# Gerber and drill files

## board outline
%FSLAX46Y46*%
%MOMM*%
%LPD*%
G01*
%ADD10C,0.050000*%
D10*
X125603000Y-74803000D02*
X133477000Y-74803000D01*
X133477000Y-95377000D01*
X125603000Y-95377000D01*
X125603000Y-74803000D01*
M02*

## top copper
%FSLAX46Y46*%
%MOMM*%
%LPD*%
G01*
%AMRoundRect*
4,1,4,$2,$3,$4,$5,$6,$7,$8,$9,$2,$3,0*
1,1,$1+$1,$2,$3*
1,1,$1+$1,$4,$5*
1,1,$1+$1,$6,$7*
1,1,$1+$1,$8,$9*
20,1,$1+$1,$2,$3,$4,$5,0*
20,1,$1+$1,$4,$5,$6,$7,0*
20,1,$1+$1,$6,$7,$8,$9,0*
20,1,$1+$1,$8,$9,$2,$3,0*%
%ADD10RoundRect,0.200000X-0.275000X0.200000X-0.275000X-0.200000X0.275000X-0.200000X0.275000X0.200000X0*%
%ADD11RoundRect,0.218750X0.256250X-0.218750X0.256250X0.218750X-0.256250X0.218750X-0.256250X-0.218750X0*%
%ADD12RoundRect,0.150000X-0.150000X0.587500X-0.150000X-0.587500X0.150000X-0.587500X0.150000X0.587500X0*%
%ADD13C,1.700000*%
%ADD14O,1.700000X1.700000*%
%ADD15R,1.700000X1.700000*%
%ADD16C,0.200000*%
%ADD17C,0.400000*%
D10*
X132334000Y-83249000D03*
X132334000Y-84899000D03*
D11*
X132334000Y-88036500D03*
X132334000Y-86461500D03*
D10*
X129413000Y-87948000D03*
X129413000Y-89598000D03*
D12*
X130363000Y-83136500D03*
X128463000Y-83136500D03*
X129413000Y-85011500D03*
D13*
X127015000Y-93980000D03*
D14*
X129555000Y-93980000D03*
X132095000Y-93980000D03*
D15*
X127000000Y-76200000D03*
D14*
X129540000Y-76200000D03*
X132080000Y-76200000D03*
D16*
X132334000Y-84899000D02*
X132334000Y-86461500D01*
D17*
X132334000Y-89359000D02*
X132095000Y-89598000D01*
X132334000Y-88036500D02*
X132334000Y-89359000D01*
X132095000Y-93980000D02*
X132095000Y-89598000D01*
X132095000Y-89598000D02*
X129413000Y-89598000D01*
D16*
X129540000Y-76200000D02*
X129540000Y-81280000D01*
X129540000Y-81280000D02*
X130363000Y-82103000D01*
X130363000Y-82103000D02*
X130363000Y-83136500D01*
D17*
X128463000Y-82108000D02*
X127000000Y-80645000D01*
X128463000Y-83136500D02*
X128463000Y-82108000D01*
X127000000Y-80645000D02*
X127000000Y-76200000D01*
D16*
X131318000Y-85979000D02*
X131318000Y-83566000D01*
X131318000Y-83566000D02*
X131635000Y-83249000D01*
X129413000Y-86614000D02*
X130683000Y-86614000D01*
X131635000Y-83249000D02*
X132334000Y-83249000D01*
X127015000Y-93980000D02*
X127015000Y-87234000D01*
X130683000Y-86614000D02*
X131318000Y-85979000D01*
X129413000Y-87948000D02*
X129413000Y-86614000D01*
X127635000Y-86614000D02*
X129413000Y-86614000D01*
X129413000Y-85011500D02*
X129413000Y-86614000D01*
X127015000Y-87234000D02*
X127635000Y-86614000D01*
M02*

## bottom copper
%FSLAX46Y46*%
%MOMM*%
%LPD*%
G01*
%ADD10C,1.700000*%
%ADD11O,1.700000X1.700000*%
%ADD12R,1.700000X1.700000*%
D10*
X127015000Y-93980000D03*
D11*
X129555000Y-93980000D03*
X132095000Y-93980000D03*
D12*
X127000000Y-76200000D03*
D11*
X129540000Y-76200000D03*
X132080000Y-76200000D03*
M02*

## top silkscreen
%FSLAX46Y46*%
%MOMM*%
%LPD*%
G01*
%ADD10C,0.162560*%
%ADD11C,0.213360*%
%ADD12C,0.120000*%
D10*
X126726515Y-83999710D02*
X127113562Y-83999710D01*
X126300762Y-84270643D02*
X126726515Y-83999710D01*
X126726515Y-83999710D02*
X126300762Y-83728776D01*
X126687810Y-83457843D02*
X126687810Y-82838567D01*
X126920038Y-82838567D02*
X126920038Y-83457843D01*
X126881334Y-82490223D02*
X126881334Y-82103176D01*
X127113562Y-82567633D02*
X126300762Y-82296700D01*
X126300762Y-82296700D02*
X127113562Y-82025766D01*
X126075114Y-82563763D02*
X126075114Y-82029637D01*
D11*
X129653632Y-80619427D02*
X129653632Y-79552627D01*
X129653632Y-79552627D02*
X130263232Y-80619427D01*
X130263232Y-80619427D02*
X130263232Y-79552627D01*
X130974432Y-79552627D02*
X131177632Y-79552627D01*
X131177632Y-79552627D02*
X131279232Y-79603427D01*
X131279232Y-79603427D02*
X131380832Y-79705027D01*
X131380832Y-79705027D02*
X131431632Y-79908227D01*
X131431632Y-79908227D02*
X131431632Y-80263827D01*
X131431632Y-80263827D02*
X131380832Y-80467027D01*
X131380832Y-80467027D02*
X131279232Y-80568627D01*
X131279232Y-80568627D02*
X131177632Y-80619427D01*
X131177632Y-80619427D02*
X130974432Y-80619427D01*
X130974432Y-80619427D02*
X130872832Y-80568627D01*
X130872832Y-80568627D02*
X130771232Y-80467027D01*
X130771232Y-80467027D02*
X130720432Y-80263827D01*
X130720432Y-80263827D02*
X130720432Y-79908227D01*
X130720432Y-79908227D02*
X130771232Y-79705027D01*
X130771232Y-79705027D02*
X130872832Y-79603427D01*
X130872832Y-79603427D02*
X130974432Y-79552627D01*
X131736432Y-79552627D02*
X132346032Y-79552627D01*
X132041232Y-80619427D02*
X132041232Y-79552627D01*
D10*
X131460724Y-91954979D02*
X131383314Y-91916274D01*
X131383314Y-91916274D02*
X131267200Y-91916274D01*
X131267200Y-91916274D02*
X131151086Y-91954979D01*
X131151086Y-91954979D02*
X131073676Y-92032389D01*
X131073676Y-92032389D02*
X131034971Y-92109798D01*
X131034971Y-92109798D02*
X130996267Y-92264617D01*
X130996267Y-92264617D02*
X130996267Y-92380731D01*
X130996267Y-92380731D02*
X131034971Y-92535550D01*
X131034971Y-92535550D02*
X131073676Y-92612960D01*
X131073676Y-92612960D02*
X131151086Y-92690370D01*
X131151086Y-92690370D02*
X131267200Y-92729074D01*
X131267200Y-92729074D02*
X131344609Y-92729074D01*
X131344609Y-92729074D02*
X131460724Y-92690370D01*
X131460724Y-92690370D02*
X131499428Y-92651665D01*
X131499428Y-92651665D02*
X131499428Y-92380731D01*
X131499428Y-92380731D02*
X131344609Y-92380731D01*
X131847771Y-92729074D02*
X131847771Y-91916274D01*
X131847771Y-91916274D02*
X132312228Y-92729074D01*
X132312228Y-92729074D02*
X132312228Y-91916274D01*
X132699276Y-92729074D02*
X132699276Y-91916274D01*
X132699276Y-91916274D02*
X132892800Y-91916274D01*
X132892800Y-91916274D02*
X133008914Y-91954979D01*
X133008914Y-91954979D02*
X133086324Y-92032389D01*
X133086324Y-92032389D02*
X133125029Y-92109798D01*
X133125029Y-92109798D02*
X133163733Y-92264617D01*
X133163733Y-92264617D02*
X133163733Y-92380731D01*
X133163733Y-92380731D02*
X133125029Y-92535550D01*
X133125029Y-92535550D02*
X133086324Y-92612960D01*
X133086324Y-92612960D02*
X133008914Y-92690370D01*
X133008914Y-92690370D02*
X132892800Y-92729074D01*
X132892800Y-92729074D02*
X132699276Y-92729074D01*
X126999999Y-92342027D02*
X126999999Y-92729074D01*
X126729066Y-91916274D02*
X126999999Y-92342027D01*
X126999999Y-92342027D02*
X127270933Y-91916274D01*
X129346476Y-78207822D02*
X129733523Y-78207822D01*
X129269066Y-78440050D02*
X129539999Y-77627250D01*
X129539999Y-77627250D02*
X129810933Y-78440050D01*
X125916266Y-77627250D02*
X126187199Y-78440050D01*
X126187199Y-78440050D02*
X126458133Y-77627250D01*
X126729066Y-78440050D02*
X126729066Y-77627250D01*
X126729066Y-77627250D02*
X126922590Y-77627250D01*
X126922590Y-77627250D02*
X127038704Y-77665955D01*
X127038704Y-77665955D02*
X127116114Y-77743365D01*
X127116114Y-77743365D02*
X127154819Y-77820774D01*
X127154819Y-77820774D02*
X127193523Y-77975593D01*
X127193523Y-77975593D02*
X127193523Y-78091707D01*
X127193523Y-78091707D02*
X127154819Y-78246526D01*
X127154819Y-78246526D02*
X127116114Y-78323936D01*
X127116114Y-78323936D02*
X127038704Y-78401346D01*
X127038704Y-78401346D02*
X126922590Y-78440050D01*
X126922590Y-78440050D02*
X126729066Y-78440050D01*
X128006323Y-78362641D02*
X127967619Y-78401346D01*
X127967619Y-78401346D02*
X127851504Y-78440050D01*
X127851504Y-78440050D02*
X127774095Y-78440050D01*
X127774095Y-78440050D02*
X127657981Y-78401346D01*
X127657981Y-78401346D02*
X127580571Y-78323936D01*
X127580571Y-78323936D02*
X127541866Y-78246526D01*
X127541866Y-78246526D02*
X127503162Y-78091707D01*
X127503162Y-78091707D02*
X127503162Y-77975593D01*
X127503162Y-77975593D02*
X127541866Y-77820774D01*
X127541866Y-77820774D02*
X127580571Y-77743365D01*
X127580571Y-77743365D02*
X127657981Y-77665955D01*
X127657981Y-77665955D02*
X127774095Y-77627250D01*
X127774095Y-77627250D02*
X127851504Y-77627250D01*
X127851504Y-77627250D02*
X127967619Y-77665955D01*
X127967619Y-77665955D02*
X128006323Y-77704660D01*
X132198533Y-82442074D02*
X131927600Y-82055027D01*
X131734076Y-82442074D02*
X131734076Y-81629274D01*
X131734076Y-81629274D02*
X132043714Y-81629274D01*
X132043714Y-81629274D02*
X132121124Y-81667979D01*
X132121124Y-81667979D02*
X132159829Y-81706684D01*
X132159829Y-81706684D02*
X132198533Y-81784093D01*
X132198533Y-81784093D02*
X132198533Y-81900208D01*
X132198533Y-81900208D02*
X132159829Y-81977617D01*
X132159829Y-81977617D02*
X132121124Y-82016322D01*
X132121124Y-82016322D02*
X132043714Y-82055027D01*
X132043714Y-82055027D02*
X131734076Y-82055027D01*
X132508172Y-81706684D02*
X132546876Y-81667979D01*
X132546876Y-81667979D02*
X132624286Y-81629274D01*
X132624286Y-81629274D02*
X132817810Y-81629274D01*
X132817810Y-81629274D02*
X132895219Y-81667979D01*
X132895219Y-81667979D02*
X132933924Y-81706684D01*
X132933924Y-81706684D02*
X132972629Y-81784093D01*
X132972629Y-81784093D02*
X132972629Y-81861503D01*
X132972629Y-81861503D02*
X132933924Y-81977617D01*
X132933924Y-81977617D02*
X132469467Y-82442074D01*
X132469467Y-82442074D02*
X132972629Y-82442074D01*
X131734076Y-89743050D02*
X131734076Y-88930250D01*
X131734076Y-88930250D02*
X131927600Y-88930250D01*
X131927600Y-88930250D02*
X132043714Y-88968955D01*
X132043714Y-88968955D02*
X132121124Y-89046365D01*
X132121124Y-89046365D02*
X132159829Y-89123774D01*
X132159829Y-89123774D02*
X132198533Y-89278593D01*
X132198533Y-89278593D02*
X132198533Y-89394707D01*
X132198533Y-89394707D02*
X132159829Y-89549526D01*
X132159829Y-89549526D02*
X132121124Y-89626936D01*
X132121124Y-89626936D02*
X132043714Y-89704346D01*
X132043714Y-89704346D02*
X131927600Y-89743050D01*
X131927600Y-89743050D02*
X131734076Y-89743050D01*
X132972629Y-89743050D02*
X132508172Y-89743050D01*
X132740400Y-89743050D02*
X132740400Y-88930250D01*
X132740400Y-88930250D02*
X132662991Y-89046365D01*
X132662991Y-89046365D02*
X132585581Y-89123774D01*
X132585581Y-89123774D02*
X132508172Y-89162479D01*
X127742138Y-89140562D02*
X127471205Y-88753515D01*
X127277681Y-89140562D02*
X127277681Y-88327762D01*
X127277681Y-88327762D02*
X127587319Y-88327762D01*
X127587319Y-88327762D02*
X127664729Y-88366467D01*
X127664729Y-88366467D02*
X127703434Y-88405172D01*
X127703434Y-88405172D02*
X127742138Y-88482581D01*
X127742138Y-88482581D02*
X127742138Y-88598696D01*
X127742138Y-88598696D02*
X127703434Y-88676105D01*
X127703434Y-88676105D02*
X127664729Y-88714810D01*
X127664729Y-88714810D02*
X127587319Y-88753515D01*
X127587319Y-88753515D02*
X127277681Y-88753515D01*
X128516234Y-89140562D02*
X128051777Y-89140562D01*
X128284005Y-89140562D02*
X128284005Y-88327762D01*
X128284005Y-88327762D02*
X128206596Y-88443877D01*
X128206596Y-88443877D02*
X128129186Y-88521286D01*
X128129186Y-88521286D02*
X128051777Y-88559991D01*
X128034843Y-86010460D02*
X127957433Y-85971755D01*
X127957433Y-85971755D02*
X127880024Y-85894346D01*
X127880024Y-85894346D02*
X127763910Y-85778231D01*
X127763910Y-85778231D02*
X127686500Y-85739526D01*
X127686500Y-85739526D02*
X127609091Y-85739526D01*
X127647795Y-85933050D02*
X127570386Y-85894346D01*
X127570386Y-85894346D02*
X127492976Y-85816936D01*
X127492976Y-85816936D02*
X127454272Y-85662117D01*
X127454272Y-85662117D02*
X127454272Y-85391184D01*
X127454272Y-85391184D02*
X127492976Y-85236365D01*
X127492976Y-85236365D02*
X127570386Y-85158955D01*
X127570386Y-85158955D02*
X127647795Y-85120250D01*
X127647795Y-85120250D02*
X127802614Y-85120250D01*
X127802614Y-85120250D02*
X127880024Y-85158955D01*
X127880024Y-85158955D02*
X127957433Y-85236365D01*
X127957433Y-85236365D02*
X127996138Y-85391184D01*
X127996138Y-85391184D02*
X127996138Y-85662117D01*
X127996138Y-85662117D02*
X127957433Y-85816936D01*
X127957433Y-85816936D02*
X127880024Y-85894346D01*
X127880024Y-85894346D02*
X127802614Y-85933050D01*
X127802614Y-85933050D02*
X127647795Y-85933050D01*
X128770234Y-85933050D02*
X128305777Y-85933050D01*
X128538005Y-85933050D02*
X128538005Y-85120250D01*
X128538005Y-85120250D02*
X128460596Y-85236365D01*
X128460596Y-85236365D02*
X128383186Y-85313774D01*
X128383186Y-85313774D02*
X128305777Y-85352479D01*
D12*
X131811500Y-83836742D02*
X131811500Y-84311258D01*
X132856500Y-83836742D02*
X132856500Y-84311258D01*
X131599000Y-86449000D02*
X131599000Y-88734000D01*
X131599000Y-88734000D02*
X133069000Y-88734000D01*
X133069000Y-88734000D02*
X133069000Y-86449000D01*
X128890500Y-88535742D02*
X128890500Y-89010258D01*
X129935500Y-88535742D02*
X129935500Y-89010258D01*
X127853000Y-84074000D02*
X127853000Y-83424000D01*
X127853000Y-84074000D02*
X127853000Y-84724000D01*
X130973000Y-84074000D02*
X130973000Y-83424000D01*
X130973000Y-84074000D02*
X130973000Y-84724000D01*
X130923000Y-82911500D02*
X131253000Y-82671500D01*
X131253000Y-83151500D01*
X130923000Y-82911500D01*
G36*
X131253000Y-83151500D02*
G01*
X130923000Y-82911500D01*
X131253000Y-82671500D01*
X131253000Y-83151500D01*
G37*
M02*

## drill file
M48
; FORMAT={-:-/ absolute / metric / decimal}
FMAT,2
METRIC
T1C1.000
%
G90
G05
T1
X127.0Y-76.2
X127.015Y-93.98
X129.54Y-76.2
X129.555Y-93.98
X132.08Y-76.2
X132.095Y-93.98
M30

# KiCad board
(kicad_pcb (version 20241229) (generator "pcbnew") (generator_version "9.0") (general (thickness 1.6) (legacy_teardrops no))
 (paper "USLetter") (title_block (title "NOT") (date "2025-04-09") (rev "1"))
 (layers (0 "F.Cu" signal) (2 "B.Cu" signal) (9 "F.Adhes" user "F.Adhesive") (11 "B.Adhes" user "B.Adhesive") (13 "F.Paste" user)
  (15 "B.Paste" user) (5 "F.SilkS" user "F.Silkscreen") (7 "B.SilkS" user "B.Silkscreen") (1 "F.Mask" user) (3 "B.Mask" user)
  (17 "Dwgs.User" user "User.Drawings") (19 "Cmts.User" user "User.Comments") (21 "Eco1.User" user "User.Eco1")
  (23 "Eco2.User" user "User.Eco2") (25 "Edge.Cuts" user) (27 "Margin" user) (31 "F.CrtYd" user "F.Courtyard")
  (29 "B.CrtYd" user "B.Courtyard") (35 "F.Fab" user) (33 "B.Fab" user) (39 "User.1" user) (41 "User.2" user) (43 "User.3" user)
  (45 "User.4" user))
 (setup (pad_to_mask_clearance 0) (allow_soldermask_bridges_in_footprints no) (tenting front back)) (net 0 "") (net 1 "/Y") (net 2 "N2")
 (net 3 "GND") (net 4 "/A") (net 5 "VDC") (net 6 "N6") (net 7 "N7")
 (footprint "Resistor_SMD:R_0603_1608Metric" (layer "F.Cu") (at 132.334 84.074 -90)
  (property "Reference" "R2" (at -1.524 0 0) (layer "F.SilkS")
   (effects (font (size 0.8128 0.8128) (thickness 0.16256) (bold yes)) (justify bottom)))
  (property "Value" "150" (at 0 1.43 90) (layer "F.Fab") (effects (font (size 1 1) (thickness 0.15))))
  (fp_line (start -0.237258 0.5225) (end 0.237258 0.5225) (stroke (width 0.12) (type solid)) (layer "F.SilkS"))
  (fp_line (start -0.237258 -0.5225) (end 0.237258 -0.5225) (stroke (width 0.12) (type solid)) (layer "F.SilkS"))
  (pad "1" smd roundrect (at -0.825 0 270) (size 0.8 0.95) (layers "F.Cu" "F.Mask" "F.Paste") (roundrect_rratio 0.25) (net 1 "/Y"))
  (pad "2" smd roundrect (at 0.825 0 270) (size 0.8 0.95) (layers "F.Cu" "F.Mask" "F.Paste") (roundrect_rratio 0.25) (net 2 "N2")))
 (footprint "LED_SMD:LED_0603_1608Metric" (layer "F.Cu") (at 132.334 87.249 90)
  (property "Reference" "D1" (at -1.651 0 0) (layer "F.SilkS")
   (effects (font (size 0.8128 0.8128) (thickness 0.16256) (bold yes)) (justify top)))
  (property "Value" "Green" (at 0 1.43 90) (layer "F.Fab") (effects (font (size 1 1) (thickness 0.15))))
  (fp_line (start 0.8 -0.735) (end -1.485 -0.735) (stroke (width 0.12) (type solid)) (layer "F.SilkS"))
  (fp_line (start -1.485 -0.735) (end -1.485 0.735) (stroke (width 0.12) (type solid)) (layer "F.SilkS"))
  (fp_line (start -1.485 0.735) (end 0.8 0.735) (stroke (width 0.12) (type solid)) (layer "F.SilkS"))
  (pad "1" smd roundrect (at -0.7875 0 90) (size 0.875 0.95) (layers "F.Cu" "F.Mask" "F.Paste") (roundrect_rratio 0.25) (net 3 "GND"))
  (pad "2" smd roundrect (at 0.7875 0 90) (size 0.875 0.95) (layers "F.Cu" "F.Mask" "F.Paste") (roundrect_rratio 0.25) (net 2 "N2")))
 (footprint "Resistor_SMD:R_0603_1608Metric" (layer "F.Cu") (at 129.413 88.773 -90)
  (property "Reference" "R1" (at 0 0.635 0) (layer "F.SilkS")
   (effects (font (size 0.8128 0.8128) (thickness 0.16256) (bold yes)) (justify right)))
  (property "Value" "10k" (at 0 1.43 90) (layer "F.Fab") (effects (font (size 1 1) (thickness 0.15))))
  (fp_line (start -0.237258 0.5225) (end 0.237258 0.5225) (stroke (width 0.12) (type solid)) (layer "F.SilkS"))
  (fp_line (start -0.237258 -0.5225) (end 0.237258 -0.5225) (stroke (width 0.12) (type solid)) (layer "F.SilkS"))
  (pad "1" smd roundrect (at -0.825 0 270) (size 0.8 0.95) (layers "F.Cu" "F.Mask" "F.Paste") (roundrect_rratio 0.25) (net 1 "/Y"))
  (pad "2" smd roundrect (at 0.825 0 270) (size 0.8 0.95) (layers "F.Cu" "F.Mask" "F.Paste") (roundrect_rratio 0.25) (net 3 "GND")))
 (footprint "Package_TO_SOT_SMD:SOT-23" (layer "F.Cu") (at 129.413 84.074 -90)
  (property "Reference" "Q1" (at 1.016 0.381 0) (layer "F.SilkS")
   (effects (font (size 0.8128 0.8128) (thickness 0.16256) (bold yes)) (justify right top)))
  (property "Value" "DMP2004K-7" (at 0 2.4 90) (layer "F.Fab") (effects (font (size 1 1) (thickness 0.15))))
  (fp_line (start 0 1.56) (end -0.65 1.56) (stroke (width 0.12) (type solid)) (layer "F.SilkS"))
  (fp_line (start 0 1.56) (end 0.65 1.56) (stroke (width 0.12) (type solid)) (layer "F.SilkS"))
  (fp_line (start 0 -1.56) (end -0.65 -1.56) (stroke (width 0.12) (type solid)) (layer "F.SilkS"))
  (fp_line (start 0 -1.56) (end 0.65 -1.56) (stroke (width 0.12) (type solid)) (layer "F.SilkS"))
  (fp_poly
   (pts (xy -1.1625 -1.51) (xy -1.4025 -1.84) (xy -0.9225 -1.84) (xy -1.1625 -1.51)) (stroke (width 0.12) (type solid)) (fill yes)
   (layer "F.SilkS"))
  (pad "1" smd roundrect (at -0.9375 -0.95 270) (size 1.475 0.6) (layers "F.Cu" "F.Mask" "F.Paste") (roundrect_rratio 0.25) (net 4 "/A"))
  (pad "2" smd roundrect (at -0.9375 0.95 270) (size 1.475 0.6) (layers "F.Cu" "F.Mask" "F.Paste") (roundrect_rratio 0.25) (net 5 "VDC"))
  (pad "3" smd roundrect (at 0.9375 0 270) (size 1.475 0.6) (layers "F.Cu" "F.Mask" "F.Paste") (roundrect_rratio 0.25) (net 1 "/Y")))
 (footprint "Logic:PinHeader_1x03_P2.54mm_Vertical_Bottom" (layer "B.Cu") (at 127.015 93.98 -90)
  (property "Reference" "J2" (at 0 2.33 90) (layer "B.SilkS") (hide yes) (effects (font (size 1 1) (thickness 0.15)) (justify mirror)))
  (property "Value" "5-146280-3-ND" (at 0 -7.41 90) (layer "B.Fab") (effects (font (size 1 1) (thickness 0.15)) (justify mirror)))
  (pad "1" thru_hole circle (at 0 0 270) (size 1.7 1.7) (drill 1) (layers "*.Cu" "*.Mask") (remove_unused_layers no) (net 1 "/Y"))
  (pad "2" thru_hole oval (at 0 -2.54 270) (size 1.7 1.7) (drill 1) (layers "*.Cu" "*.Mask") (remove_unused_layers no) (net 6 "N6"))
  (pad "3" thru_hole oval (at 0 -5.08 270) (size 1.7 1.7) (drill 1) (layers "*.Cu" "*.Mask") (remove_unused_layers no) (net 3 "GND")))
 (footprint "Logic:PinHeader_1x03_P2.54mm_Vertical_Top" (layer "B.Cu") (at 127 76.2 -90)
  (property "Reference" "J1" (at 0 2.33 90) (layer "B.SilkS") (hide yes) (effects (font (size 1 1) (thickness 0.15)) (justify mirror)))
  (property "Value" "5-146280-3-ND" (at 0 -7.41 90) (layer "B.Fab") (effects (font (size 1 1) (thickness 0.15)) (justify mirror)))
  (pad "1" thru_hole rect (at 0 0 270) (size 1.7 1.7) (drill 1) (layers "*.Cu" "*.Mask") (remove_unused_layers no) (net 5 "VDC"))
  (pad "2" thru_hole oval (at 0 -2.54 270) (size 1.7 1.7) (drill 1) (layers "*.Cu" "*.Mask") (remove_unused_layers no) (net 4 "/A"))
  (pad "3" thru_hole oval (at 0 -5.08 270) (size 1.7 1.7) (drill 1) (layers "*.Cu" "*.Mask") (remove_unused_layers no) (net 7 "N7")))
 (gr_rect (start 125.603 74.803) (end 133.477 95.377) (stroke (width 0.05) (type default)) (fill no) (layer "Edge.Cuts"))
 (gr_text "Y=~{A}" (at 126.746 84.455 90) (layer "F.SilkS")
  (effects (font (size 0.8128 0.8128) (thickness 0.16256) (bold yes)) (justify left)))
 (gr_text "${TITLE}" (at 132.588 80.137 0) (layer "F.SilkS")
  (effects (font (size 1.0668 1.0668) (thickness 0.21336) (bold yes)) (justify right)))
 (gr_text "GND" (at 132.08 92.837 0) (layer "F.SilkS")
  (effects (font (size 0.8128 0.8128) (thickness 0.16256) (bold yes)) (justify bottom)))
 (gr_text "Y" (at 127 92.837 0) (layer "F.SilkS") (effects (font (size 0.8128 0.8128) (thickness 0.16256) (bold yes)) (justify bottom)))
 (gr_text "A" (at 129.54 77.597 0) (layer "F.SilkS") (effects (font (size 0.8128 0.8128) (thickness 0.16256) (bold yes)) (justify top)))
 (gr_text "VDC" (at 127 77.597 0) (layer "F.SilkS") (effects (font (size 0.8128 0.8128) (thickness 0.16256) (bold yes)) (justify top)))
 (segment (start 132.334 84.899) (end 132.334 86.4615) (width 0.2) (layer "F.Cu") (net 2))
 (segment (start 132.334 89.359) (end 132.095 89.598) (width 0.4) (layer "F.Cu") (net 3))
 (segment (start 132.334 88.0365) (end 132.334 89.359) (width 0.4) (layer "F.Cu") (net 3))
 (segment (start 132.095 93.98) (end 132.095 89.598) (width 0.4) (layer "F.Cu") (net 3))
 (segment (start 132.095 89.598) (end 129.413 89.598) (width 0.4) (layer "F.Cu") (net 3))
 (segment (start 129.54 76.2) (end 129.54 81.28) (width 0.2) (layer "F.Cu") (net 4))
 (segment (start 129.54 81.28) (end 130.363 82.103) (width 0.2) (layer "F.Cu") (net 4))
 (segment (start 130.363 82.103) (end 130.363 83.1365) (width 0.2) (layer "F.Cu") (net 4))
 (segment (start 128.463 82.108) (end 127 80.645) (width 0.4) (layer "F.Cu") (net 5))
 (segment (start 128.463 83.1365) (end 128.463 82.108) (width 0.4) (layer "F.Cu") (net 5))
 (segment (start 127 80.645) (end 127 76.2) (width 0.4) (layer "F.Cu") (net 5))
 (segment (start 131.318 85.979) (end 131.318 83.566) (width 0.2) (layer "F.Cu") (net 1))
 (segment (start 131.318 83.566) (end 131.635 83.249) (width 0.2) (layer "F.Cu") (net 1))
 (segment (start 129.413 86.614) (end 130.683 86.614) (width 0.2) (layer "F.Cu") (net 1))
 (segment (start 131.635 83.249) (end 132.334 83.249) (width 0.2) (layer "F.Cu") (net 1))
 (segment (start 127.015 93.98) (end 127.015 87.234) (width 0.2) (layer "F.Cu") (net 1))
 (segment (start 130.683 86.614) (end 131.318 85.979) (width 0.2) (layer "F.Cu") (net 1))
 (segment (start 129.413 87.948) (end 129.413 86.614) (width 0.2) (layer "F.Cu") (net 1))
 (segment (start 127.635 86.614) (end 129.413 86.614) (width 0.2) (layer "F.Cu") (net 1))
 (segment (start 129.413 85.0115) (end 129.413 86.614) (width 0.2) (layer "F.Cu") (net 1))
 (segment (start 127.015 87.234) (end 127.635 86.614) (width 0.2) (layer "F.Cu") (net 1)))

